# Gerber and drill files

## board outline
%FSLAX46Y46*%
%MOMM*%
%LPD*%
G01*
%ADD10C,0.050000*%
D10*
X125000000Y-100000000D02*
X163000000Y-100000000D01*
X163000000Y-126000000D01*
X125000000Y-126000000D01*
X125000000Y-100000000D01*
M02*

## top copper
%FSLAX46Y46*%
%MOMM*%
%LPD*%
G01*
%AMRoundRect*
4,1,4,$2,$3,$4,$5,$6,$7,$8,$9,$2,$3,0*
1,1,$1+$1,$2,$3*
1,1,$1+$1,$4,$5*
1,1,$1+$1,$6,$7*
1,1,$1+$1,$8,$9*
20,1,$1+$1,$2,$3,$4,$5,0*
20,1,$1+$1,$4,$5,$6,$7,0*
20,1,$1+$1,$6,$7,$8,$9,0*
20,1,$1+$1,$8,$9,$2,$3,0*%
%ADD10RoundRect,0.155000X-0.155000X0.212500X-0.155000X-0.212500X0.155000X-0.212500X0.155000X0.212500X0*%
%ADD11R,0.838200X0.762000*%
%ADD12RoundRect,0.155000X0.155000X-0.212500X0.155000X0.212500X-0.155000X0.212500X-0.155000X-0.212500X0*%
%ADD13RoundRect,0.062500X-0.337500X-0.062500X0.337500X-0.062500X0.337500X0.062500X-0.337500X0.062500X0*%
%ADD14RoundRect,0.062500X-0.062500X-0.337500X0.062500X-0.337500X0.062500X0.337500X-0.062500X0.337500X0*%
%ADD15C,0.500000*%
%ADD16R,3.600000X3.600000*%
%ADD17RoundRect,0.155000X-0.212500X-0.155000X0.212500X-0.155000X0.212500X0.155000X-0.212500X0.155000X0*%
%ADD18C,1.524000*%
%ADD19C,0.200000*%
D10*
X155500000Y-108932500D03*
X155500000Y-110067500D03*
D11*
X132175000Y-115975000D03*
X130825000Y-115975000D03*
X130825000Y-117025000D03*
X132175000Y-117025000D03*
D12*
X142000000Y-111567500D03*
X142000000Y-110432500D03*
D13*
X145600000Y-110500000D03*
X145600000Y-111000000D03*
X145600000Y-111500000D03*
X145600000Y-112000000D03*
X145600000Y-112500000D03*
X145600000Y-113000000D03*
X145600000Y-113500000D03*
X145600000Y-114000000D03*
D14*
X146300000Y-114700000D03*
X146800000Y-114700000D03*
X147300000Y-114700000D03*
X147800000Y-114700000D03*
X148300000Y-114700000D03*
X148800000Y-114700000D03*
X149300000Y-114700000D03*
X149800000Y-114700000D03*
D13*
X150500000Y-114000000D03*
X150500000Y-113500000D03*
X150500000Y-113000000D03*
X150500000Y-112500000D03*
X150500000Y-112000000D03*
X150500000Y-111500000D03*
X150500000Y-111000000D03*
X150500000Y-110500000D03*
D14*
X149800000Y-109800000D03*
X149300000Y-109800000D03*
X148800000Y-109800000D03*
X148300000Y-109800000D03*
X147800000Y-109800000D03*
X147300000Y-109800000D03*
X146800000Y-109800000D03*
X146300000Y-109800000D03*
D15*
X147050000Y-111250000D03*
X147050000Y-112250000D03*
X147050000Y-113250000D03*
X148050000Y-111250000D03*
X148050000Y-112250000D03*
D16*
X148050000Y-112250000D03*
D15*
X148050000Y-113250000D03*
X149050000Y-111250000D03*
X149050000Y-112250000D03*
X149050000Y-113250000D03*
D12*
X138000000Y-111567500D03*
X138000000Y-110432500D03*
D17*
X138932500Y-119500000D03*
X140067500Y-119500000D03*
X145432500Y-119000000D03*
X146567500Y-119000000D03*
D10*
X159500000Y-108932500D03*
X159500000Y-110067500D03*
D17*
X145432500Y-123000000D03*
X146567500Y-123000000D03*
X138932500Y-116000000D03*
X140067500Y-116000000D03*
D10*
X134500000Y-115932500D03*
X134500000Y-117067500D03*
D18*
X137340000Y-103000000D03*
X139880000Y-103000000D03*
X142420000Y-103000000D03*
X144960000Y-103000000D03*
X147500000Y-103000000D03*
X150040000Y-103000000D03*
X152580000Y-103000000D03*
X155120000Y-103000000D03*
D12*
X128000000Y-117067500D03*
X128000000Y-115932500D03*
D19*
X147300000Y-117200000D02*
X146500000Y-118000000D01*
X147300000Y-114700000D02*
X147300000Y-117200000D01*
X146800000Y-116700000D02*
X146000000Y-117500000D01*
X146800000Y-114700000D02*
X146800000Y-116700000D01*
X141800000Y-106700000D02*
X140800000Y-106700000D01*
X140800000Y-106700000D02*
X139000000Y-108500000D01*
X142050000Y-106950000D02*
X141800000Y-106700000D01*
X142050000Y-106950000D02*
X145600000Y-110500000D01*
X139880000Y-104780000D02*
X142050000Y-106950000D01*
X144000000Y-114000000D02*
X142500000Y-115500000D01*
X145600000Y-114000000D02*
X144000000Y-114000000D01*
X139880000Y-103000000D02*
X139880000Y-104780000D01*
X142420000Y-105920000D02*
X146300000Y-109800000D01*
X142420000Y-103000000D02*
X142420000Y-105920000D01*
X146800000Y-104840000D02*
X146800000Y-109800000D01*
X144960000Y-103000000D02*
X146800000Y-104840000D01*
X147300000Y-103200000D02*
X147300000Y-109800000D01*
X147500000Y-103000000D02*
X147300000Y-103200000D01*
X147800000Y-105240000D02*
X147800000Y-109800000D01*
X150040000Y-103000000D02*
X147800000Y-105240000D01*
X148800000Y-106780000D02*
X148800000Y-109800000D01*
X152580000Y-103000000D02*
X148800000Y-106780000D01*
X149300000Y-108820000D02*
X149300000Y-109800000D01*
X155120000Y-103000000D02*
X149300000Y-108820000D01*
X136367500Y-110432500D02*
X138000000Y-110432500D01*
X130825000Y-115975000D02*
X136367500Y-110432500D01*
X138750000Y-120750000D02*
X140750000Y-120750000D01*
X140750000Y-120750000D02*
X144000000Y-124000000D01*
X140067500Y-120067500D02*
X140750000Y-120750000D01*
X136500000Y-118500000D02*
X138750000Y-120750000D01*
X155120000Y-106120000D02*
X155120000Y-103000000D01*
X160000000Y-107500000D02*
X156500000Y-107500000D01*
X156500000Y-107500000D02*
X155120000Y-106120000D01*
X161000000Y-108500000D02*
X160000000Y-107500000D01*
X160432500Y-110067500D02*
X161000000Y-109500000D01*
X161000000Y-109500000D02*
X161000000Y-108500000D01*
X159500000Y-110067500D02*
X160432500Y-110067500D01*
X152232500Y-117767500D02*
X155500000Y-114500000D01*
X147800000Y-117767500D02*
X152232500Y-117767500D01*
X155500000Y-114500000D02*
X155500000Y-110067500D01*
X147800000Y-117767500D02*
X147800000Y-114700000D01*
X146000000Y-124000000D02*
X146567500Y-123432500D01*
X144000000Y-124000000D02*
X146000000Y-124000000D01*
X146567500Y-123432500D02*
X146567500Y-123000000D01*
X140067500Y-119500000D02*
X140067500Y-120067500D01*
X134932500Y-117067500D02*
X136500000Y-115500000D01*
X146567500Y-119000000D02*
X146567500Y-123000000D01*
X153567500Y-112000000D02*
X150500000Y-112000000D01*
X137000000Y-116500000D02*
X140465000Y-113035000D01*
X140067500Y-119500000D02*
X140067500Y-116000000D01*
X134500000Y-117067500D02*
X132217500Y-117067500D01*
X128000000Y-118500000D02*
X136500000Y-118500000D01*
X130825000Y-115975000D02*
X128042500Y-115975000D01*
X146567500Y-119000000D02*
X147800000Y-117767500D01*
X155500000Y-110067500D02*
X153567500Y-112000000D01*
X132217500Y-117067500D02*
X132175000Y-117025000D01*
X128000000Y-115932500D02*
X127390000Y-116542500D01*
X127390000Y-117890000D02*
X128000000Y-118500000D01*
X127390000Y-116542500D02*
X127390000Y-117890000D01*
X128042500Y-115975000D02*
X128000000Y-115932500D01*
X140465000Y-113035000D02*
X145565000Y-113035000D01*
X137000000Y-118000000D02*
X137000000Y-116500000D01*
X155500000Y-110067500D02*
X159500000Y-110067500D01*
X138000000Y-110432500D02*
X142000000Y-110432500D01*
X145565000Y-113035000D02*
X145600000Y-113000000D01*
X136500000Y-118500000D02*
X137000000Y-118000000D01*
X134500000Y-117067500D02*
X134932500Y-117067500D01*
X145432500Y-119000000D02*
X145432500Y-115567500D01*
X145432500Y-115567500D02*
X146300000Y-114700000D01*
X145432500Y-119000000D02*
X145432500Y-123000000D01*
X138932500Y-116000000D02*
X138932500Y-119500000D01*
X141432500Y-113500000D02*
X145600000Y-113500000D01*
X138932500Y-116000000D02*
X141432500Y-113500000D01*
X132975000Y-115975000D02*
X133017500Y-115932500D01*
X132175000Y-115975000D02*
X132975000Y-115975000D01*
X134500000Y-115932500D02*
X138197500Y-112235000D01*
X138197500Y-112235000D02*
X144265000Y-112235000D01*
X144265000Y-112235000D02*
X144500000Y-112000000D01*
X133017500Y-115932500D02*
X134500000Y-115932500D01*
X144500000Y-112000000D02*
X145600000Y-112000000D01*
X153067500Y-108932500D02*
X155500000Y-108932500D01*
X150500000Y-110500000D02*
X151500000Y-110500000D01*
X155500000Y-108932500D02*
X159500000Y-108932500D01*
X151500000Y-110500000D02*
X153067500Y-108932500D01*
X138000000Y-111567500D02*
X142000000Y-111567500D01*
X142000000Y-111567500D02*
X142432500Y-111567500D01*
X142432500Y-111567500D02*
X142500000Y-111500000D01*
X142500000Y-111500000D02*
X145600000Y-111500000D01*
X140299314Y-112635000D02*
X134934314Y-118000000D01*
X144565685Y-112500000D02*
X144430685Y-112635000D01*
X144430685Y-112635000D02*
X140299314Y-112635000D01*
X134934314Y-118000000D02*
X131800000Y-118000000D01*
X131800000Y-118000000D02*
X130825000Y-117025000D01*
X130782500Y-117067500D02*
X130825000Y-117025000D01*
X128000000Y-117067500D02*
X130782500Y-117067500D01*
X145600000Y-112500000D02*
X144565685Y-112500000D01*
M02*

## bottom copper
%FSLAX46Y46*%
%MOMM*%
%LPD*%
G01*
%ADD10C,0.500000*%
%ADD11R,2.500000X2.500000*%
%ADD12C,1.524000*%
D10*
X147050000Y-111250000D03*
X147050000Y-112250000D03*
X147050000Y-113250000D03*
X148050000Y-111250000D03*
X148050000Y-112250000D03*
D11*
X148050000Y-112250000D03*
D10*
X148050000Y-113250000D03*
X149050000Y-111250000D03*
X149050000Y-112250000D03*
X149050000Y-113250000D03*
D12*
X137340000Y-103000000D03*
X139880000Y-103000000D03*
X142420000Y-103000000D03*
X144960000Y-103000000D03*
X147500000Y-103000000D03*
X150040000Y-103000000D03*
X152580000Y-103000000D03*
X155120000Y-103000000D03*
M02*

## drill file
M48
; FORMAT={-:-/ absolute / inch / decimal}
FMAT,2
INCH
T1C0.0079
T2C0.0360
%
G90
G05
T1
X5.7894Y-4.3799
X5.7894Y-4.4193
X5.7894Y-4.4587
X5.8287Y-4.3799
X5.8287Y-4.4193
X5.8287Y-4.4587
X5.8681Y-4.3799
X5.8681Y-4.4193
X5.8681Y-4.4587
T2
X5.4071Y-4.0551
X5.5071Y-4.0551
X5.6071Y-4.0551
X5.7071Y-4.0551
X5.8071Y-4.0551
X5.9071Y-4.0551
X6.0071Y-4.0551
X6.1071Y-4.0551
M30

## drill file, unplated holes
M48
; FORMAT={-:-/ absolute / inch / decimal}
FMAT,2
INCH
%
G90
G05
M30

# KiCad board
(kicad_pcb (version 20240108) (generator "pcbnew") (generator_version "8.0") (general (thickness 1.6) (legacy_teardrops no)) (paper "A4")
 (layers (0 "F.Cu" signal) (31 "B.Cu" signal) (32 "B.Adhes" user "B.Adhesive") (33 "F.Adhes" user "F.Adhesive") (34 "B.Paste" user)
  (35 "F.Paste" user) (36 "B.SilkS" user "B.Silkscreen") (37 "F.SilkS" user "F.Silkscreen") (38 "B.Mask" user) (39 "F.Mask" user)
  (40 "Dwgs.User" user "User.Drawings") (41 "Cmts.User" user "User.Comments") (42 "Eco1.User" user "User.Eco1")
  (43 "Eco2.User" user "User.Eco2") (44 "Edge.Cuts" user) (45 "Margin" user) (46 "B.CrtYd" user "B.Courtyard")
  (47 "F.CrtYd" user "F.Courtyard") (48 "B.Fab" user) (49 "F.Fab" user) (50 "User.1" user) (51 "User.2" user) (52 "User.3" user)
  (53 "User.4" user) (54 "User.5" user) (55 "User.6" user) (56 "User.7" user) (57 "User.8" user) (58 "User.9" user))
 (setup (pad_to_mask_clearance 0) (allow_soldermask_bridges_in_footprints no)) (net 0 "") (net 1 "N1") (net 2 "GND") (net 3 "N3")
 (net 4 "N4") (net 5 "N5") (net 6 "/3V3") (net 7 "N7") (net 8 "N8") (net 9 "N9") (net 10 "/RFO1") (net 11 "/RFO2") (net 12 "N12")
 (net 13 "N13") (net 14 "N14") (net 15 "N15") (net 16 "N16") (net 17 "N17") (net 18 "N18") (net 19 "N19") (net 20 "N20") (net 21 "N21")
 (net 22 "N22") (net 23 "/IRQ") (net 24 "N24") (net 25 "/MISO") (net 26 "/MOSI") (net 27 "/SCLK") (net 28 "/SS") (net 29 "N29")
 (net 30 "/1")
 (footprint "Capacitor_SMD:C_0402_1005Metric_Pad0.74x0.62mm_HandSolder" (layer "F.Cu") (at 155.5 109.5 -90)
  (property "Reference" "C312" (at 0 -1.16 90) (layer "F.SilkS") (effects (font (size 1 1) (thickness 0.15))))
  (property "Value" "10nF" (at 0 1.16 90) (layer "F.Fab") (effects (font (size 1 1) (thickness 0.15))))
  (pad "1" smd roundrect (at -0.5675 0 270) (size 0.735 0.62) (layers "F.Cu" "F.Paste" "F.Mask") (roundrect_rratio 0.25) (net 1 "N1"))
  (pad "2" smd roundrect (at 0.5675 0 270) (size 0.735 0.62) (layers "F.Cu" "F.Paste" "F.Mask") (roundrect_rratio 0.25) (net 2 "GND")))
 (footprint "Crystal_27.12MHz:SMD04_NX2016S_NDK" (layer "F.Cu") (at 131.5 116.5 -90)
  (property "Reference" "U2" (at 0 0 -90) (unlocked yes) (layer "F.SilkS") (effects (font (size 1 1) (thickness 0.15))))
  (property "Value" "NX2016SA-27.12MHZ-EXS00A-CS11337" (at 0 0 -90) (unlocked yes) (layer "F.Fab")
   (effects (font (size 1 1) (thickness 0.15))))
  (pad "1" smd rect (at -0.525 -0.675 270) (size 0.762 0.8382) (layers "F.Cu" "F.Paste" "F.Mask") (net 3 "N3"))
  (pad "2" smd rect (at -0.525 0.675 270) (size 0.762 0.8382) (layers "F.Cu" "F.Paste" "F.Mask") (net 2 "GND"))
  (pad "3" smd rect (at 0.525 0.675 270) (size 0.762 0.8382) (layers "F.Cu" "F.Paste" "F.Mask") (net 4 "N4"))
  (pad "4" smd rect (at 0.525 -0.675 270) (size 0.762 0.8382) (layers "F.Cu" "F.Paste" "F.Mask") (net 2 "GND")))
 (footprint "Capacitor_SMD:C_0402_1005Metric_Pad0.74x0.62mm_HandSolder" (layer "F.Cu") (at 142 111 90)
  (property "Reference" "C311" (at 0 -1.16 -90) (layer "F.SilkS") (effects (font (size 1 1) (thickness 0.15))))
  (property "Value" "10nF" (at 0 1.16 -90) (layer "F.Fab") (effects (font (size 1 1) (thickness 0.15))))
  (pad "1" smd roundrect (at -0.5675 0 90) (size 0.735 0.62) (layers "F.Cu" "F.Paste" "F.Mask") (roundrect_rratio 0.25) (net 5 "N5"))
  (pad "2" smd roundrect (at 0.5675 0 90) (size 0.735 0.62) (layers "F.Cu" "F.Paste" "F.Mask") (roundrect_rratio 0.25) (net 2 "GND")))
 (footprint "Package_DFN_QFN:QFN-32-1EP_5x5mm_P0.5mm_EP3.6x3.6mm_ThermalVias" (layer "F.Cu") (at 148.05 112.25)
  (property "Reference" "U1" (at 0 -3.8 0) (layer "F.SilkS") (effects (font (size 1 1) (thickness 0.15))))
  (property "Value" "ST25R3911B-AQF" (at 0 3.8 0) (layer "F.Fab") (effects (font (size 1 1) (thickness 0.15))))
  (pad "" smd custom (at -1.4 -1.4) (size 0.554596 0.554596) (layers "F.Paste") (options (clearance outline) (anchor circle)) (primitives))
  (pad "" smd custom (at -1.4 -0.5) (size 0.568298 0.568298) (layers "F.Paste") (options (clearance outline) (anchor circle)) (primitives))
  (pad "" smd custom (at -1.4 0.5) (size 0.568298 0.568298) (layers "F.Paste") (options (clearance outline) (anchor circle)) (primitives))
  (pad "" smd custom (at -1.4 1.4) (size 0.554596 0.554596) (layers "F.Paste") (options (clearance outline) (anchor circle)) (primitives))
  (pad "" smd custom (at -0.5 -1.4) (size 0.568298 0.568298) (layers "F.Paste") (options (clearance outline) (anchor circle)) (primitives))
  (pad "" smd roundrect (at -0.5 -0.5) (size 0.806226 0.806226) (layers "F.Paste") (roundrect_rratio 0.25))
  (pad "" smd roundrect (at -0.5 0.5) (size 0.806226 0.806226) (layers "F.Paste") (roundrect_rratio 0.25))
  (pad "" smd custom (at -0.5 1.4) (size 0.568298 0.568298) (layers "F.Paste") (options (clearance outline) (anchor circle)) (primitives))
  (pad "" smd custom (at 0.5 -1.4) (size 0.568298 0.568298) (layers "F.Paste") (options (clearance outline) (anchor circle)) (primitives))
  (pad "" smd roundrect (at 0.5 -0.5) (size 0.806226 0.806226) (layers "F.Paste") (roundrect_rratio 0.25))
  (pad "" smd roundrect (at 0.5 0.5) (size 0.806226 0.806226) (layers "F.Paste") (roundrect_rratio 0.25))
  (pad "" smd custom (at 0.5 1.4) (size 0.568298 0.568298) (layers "F.Paste") (options (clearance outline) (anchor circle)) (primitives))
  (pad "" smd custom (at 1.4 -1.4) (size 0.554596 0.554596) (layers "F.Paste") (options (clearance outline) (anchor circle)) (primitives))
  (pad "" smd custom (at 1.4 -0.5) (size 0.568298 0.568298) (layers "F.Paste") (options (clearance outline) (anchor circle)) (primitives))
  (pad "" smd custom (at 1.4 0.5) (size 0.568298 0.568298) (layers "F.Paste") (options (clearance outline) (anchor circle)) (primitives))
  (pad "" smd custom (at 1.4 1.4) (size 0.554596 0.554596) (layers "F.Paste") (options (clearance outline) (anchor circle)) (primitives))
  (pad "1" smd roundrect (at -2.45 -1.75) (size 0.8 0.25) (layers "F.Cu" "F.Paste" "F.Mask") (roundrect_rratio 0.25) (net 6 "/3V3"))
  (pad "2" smd roundrect (at -2.45 -1.25) (size 0.8 0.25) (layers "F.Cu" "F.Paste" "F.Mask") (roundrect_rratio 0.25) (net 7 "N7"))
  (pad "3" smd roundrect (at -2.45 -0.75) (size 0.8 0.25) (layers "F.Cu" "F.Paste" "F.Mask") (roundrect_rratio 0.25) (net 5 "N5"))
  (pad "4" smd roundrect (at -2.45 -0.25) (size 0.8 0.25) (layers "F.Cu" "F.Paste" "F.Mask") (roundrect_rratio 0.25) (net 3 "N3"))
  (pad "5" smd roundrect (at -2.45 0.25) (size 0.8 0.25) (layers "F.Cu" "F.Paste" "F.Mask") (roundrect_rratio 0.25) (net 4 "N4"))
  (pad "6" smd roundrect (at -2.45 0.75) (size 0.8 0.25) (layers "F.Cu" "F.Paste" "F.Mask") (roundrect_rratio 0.25) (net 2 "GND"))
  (pad "7" smd roundrect (at -2.45 1.25) (size 0.8 0.25) (layers "F.Cu" "F.Paste" "F.Mask") (roundrect_rratio 0.25) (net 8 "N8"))
  (pad "8" smd roundrect (at -2.45 1.75) (size 0.8 0.25) (layers "F.Cu" "F.Paste" "F.Mask") (roundrect_rratio 0.25) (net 6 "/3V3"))
  (pad "9" smd roundrect (at -1.75 2.45) (size 0.25 0.8) (layers "F.Cu" "F.Paste" "F.Mask") (roundrect_rratio 0.25) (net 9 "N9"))
  (pad "10" smd roundrect (at -1.25 2.45) (size 0.25 0.8) (layers "F.Cu" "F.Paste" "F.Mask") (roundrect_rratio 0.25) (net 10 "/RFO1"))
  (pad "11" smd roundrect (at -0.75 2.45) (size 0.25 0.8) (layers "F.Cu" "F.Paste" "F.Mask") (roundrect_rratio 0.25) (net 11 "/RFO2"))
  (pad "12" smd roundrect (at -0.25 2.45) (size 0.25 0.8) (layers "F.Cu" "F.Paste" "F.Mask") (roundrect_rratio 0.25) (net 2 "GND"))
  (pad "13" smd roundrect (at 0.25 2.45) (size 0.25 0.8) (layers "F.Cu" "F.Paste" "F.Mask") (roundrect_rratio 0.25) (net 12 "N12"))
  (pad "14" smd roundrect (at 0.75 2.45) (size 0.25 0.8) (layers "F.Cu" "F.Paste" "F.Mask") (roundrect_rratio 0.25) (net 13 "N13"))
  (pad "15" smd roundrect (at 1.25 2.45) (size 0.25 0.8) (layers "F.Cu" "F.Paste" "F.Mask") (roundrect_rratio 0.25) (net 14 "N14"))
  (pad "16" smd roundrect (at 1.75 2.45) (size 0.25 0.8) (layers "F.Cu" "F.Paste" "F.Mask") (roundrect_rratio 0.25) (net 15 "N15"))
  (pad "17" smd roundrect (at 2.45 1.75) (size 0.8 0.25) (layers "F.Cu" "F.Paste" "F.Mask") (roundrect_rratio 0.25) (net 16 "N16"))
  (pad "18" smd roundrect (at 2.45 1.25) (size 0.8 0.25) (layers "F.Cu" "F.Paste" "F.Mask") (roundrect_rratio 0.25) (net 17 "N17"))
  (pad "19" smd roundrect (at 2.45 0.75) (size 0.8 0.25) (layers "F.Cu" "F.Paste" "F.Mask") (roundrect_rratio 0.25) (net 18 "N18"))
  (pad "20" smd roundrect (at 2.45 0.25) (size 0.8 0.25) (layers "F.Cu" "F.Paste" "F.Mask") (roundrect_rratio 0.25) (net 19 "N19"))
  (pad "21" smd roundrect (at 2.45 -0.25) (size 0.8 0.25) (layers "F.Cu" "F.Paste" "F.Mask") (roundrect_rratio 0.25) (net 2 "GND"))
  (pad "22" smd roundrect (at 2.45 -0.75) (size 0.8 0.25) (layers "F.Cu" "F.Paste" "F.Mask") (roundrect_rratio 0.25) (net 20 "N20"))
  (pad "23" smd roundrect (at 2.45 -1.25) (size 0.8 0.25) (layers "F.Cu" "F.Paste" "F.Mask") (roundrect_rratio 0.25) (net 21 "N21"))
  (pad "24" smd roundrect (at 2.45 -1.75) (size 0.8 0.25) (layers "F.Cu" "F.Paste" "F.Mask") (roundrect_rratio 0.25) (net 1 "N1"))
  (pad "25" smd roundrect (at 1.75 -2.45) (size 0.25 0.8) (layers "F.Cu" "F.Paste" "F.Mask") (roundrect_rratio 0.25) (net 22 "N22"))
  (pad "26" smd roundrect (at 1.25 -2.45) (size 0.25 0.8) (layers "F.Cu" "F.Paste" "F.Mask") (roundrect_rratio 0.25) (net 2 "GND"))
  (pad "27" smd roundrect (at 0.75 -2.45) (size 0.25 0.8) (layers "F.Cu" "F.Paste" "F.Mask") (roundrect_rratio 0.25) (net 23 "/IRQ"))
  (pad "28" smd roundrect (at 0.25 -2.45) (size 0.25 0.8) (layers "F.Cu" "F.Paste" "F.Mask") (roundrect_rratio 0.25) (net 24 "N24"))
  (pad "29" smd roundrect (at -0.25 -2.45) (size 0.25 0.8) (layers "F.Cu" "F.Paste" "F.Mask") (roundrect_rratio 0.25) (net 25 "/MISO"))
  (pad "30" smd roundrect (at -0.75 -2.45) (size 0.25 0.8) (layers "F.Cu" "F.Paste" "F.Mask") (roundrect_rratio 0.25) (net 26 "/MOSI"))
  (pad "31" smd roundrect (at -1.25 -2.45) (size 0.25 0.8) (layers "F.Cu" "F.Paste" "F.Mask") (roundrect_rratio 0.25) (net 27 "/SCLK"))
  (pad "32" smd roundrect (at -1.75 -2.45) (size 0.25 0.8) (layers "F.Cu" "F.Paste" "F.Mask") (roundrect_rratio 0.25) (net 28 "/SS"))
  (pad "33" thru_hole circle (at -1 -1) (size 0.5 0.5) (drill 0.2) (layers "*.Cu") (remove_unused_layers no) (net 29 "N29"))
  (pad "33" thru_hole circle (at -1 0) (size 0.5 0.5) (drill 0.2) (layers "*.Cu") (remove_unused_layers no) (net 29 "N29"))
  (pad "33" thru_hole circle (at -1 1) (size 0.5 0.5) (drill 0.2) (layers "*.Cu") (remove_unused_layers no) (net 29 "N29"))
  (pad "33" thru_hole circle (at 0 -1) (size 0.5 0.5) (drill 0.2) (layers "*.Cu") (remove_unused_layers no) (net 29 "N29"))
  (pad "33" thru_hole circle (at 0 0) (size 0.5 0.5) (drill 0.2) (layers "*.Cu") (remove_unused_layers no) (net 29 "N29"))
  (pad "33" smd rect (at 0 0) (size 2.5 2.5) (layers "B.Cu") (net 29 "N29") (zone_connect 2))
  (pad "33" smd rect (at 0 0) (size 3.6 3.6) (layers "F.Cu" "F.Mask") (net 29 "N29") (zone_connect 2))
  (pad "33" thru_hole circle (at 0 1) (size 0.5 0.5) (drill 0.2) (layers "*.Cu") (remove_unused_layers no) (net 29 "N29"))
  (pad "33" thru_hole circle (at 1 -1) (size 0.5 0.5) (drill 0.2) (layers "*.Cu") (remove_unused_layers no) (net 29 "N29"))
  (pad "33" thru_hole circle (at 1 0) (size 0.5 0.5) (drill 0.2) (layers "*.Cu") (remove_unused_layers no) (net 29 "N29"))
  (pad "33" thru_hole circle (at 1 1) (size 0.5 0.5) (drill 0.2) (layers "*.Cu") (remove_unused_layers no) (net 29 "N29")))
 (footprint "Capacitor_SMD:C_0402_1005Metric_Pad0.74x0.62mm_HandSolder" (layer "F.Cu") (at 138 111 90)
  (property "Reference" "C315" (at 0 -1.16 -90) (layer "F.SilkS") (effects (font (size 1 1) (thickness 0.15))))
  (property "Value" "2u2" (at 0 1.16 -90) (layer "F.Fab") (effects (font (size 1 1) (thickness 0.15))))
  (pad "1" smd roundrect (at -0.5675 0 90) (size 0.735 0.62) (layers "F.Cu" "F.Paste" "F.Mask") (roundrect_rratio 0.25) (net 5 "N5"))
  (pad "2" smd roundrect (at 0.5675 0 90) (size 0.735 0.62) (layers "F.Cu" "F.Paste" "F.Mask") (roundrect_rratio 0.25) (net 2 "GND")))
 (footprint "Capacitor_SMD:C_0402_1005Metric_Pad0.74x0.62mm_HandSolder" (layer "F.Cu") (at 139.5 119.5)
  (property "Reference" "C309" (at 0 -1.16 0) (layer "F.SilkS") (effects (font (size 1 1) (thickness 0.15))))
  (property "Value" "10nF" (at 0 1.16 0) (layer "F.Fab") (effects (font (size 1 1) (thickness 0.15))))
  (pad "1" smd roundrect (at -0.5675 0) (size 0.735 0.62) (layers "F.Cu" "F.Paste" "F.Mask") (roundrect_rratio 0.25) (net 8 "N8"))
  (pad "2" smd roundrect (at 0.5675 0) (size 0.735 0.62) (layers "F.Cu" "F.Paste" "F.Mask") (roundrect_rratio 0.25) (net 2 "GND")))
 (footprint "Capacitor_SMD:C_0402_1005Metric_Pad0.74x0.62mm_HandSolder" (layer "F.Cu") (at 146 119)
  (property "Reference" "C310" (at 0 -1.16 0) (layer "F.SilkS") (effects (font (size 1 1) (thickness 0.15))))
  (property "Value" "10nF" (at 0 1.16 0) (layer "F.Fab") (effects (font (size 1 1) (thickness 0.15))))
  (pad "1" smd roundrect (at -0.5675 0) (size 0.735 0.62) (layers "F.Cu" "F.Paste" "F.Mask") (roundrect_rratio 0.25) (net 9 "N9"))
  (pad "2" smd roundrect (at 0.5675 0) (size 0.735 0.62) (layers "F.Cu" "F.Paste" "F.Mask") (roundrect_rratio 0.25) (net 2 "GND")))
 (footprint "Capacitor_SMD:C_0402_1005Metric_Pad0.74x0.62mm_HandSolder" (layer "F.Cu") (at 159.5 109.5 -90)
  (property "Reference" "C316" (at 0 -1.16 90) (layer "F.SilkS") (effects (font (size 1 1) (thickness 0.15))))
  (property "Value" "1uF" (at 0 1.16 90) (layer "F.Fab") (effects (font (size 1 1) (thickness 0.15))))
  (pad "1" smd roundrect (at -0.5675 0 270) (size 0.735 0.62) (layers "F.Cu" "F.Paste" "F.Mask") (roundrect_rratio 0.25) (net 1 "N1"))
  (pad "2" smd roundrect (at 0.5675 0 270) (size 0.735 0.62) (layers "F.Cu" "F.Paste" "F.Mask") (roundrect_rratio 0.25) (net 2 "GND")))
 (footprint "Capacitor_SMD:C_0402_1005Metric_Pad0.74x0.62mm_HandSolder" (layer "F.Cu") (at 146 123)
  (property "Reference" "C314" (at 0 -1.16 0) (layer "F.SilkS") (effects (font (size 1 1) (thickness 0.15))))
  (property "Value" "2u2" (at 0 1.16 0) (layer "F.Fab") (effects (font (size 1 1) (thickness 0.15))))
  (pad "1" smd roundrect (at -0.5675 0) (size 0.735 0.62) (layers "F.Cu" "F.Paste" "F.Mask") (roundrect_rratio 0.25) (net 9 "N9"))
  (pad "2" smd roundrect (at 0.5675 0) (size 0.735 0.62) (layers "F.Cu" "F.Paste" "F.Mask") (roundrect_rratio 0.25) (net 2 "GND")))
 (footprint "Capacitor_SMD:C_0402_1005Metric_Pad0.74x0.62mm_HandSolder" (layer "F.Cu") (at 139.5 116)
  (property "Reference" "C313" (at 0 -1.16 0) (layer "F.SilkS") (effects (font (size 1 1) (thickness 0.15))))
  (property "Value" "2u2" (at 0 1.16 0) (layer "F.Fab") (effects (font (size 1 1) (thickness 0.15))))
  (pad "1" smd roundrect (at -0.5675 0) (size 0.735 0.62) (layers "F.Cu" "F.Paste" "F.Mask") (roundrect_rratio 0.25) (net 8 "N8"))
  (pad "2" smd roundrect (at 0.5675 0) (size 0.735 0.62) (layers "F.Cu" "F.Paste" "F.Mask") (roundrect_rratio 0.25) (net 2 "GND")))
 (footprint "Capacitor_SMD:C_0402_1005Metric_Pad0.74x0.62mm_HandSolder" (layer "F.Cu") (at 134.5 116.5 -90)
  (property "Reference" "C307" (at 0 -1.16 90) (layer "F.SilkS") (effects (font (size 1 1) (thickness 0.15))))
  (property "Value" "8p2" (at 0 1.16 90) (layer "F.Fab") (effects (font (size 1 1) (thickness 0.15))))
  (pad "1" smd roundrect (at -0.5675 0 270) (size 0.735 0.62) (layers "F.Cu" "F.Paste" "F.Mask") (roundrect_rratio 0.25) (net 3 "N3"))
  (pad "2" smd roundrect (at 0.5675 0 270) (size 0.735 0.62) (layers "F.Cu" "F.Paste" "F.Mask") (roundrect_rratio 0.25) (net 2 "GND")))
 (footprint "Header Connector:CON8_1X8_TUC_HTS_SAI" (layer "F.Cu") (at 146.23 103)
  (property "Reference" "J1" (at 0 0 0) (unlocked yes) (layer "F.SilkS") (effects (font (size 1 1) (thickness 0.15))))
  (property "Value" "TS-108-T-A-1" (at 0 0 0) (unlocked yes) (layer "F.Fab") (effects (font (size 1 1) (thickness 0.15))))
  (pad "1" thru_hole circle (at -8.89 0 90) (size 1.524 1.524) (drill 0.9144) (layers "*.Cu" "*.Mask") (remove_unused_layers no)
   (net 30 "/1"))
  (pad "2" thru_hole circle (at -6.35 0 90) (size 1.524 1.524) (drill 0.9144) (layers "*.Cu" "*.Mask") (remove_unused_layers no)
   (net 6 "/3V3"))
  (pad "3" thru_hole circle (at -3.81 0 90) (size 1.524 1.524) (drill 0.9144) (layers "*.Cu" "*.Mask") (remove_unused_layers no)
   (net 28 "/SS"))
  (pad "4" thru_hole circle (at -1.27 0 90) (size 1.524 1.524) (drill 0.9144) (layers "*.Cu" "*.Mask") (remove_unused_layers no)
   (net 27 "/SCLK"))
  (pad "5" thru_hole circle (at 1.27 0 90) (size 1.524 1.524) (drill 0.9144) (layers "*.Cu" "*.Mask") (remove_unused_layers no)
   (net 26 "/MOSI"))
  (pad "6" thru_hole circle (at 3.81 0 90) (size 1.524 1.524) (drill 0.9144) (layers "*.Cu" "*.Mask") (remove_unused_layers no)
   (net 25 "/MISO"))
  (pad "7" thru_hole circle (at 6.35 0 90) (size 1.524 1.524) (drill 0.9144) (layers "*.Cu" "*.Mask") (remove_unused_layers no)
   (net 23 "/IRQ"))
  (pad "8" thru_hole circle (at 8.89 0 90) (size 1.524 1.524) (drill 0.9144) (layers "*.Cu" "*.Mask") (remove_unused_layers no)
   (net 2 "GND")))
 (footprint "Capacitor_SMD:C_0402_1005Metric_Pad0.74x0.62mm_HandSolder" (layer "F.Cu") (at 128 116.5 90)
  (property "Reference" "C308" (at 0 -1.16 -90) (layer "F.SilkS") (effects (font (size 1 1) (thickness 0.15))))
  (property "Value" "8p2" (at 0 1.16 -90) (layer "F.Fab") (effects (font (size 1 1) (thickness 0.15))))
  (pad "1" smd roundrect (at -0.5675 0 90) (size 0.735 0.62) (layers "F.Cu" "F.Paste" "F.Mask") (roundrect_rratio 0.25) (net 4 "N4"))
  (pad "2" smd roundrect (at 0.5675 0 90) (size 0.735 0.62) (layers "F.Cu" "F.Paste" "F.Mask") (roundrect_rratio 0.25) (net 2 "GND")))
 (gr_rect (start 125 100) (end 163 126) (stroke (width 0.05) (type default)) (fill none) (layer "Edge.Cuts"))
 (segment (start 147.5 103) (end 147.3 103.2) (width 0.2) (layer "F.Cu") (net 26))
 (segment (start 147.3 103.2) (end 147.3 109.8) (width 0.2) (layer "F.Cu") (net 26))
 (segment (start 144 114) (end 142.5 115.5) (width 0.2) (layer "F.Cu") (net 6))
 (segment (start 139.88 103) (end 139.88 104.78) (width 0.2) (layer "F.Cu") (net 6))
 (segment (start 140.8 106.7) (end 139 108.5) (width 0.2) (layer "F.Cu") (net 6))
 (segment (start 139.88 104.78) (end 142.05 106.95) (width 0.2) (layer "F.Cu") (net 6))
 (segment (start 141.8 106.7) (end 140.8 106.7) (width 0.2) (layer "F.Cu") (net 6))
 (segment (start 142.05 106.95) (end 141.8 106.7) (width 0.2) (layer "F.Cu") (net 6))
 (segment (start 145.6 114) (end 144 114) (width 0.2) (layer "F.Cu") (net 6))
 (segment (start 142.05 106.95) (end 145.6 110.5) (width 0.2) (layer "F.Cu") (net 6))
 (segment (start 152.58 103) (end 148.8 106.78) (width 0.2) (layer "F.Cu") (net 23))
 (segment (start 148.8 106.78) (end 148.8 109.8) (width 0.2) (layer "F.Cu") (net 23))
 (segment (start 136.5 118.5) (end 138.75 120.75) (width 0.2) (layer "F.Cu") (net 2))
 (segment (start 134.9325 117.0675) (end 136.5 115.5) (width 0.2) (layer "F.Cu") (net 2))
 (segment (start 146.5675 119) (end 146.5675 123) (width 0.2) (layer "F.Cu") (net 2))
 (segment (start 155.12 106.12) (end 155.12 103) (width 0.2) (layer "F.Cu") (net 2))
 (segment (start 153.5675 112) (end 150.5 112) (width 0.2) (layer "F.Cu") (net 2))
 (segment (start 160.4325 110.0675) (end 161 109.5) (width 0.2) (layer "F.Cu") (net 2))
 (segment (start 137 116.5) (end 140.465 113.035) (width 0.2) (layer "F.Cu") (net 2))
 (segment (start 146 124) (end 146.5675 123.4325) (width 0.2) (layer "F.Cu") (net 2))
 (segment (start 147.8 117.7675) (end 152.2325 117.7675) (width 0.2) (layer "F.Cu") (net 2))
 (segment (start 140.0675 119.5) (end 140.0675 116) (width 0.2) (layer "F.Cu") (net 2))
 (segment (start 140.0675 120.0675) (end 140.75 120.75) (width 0.2) (layer "F.Cu") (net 2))
 (segment (start 134.5 117.0675) (end 132.2175 117.0675) (width 0.2) (layer "F.Cu") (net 2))
 (segment (start 140.75 120.75) (end 144 124) (width 0.2) (layer "F.Cu") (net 2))
 (segment (start 160 107.5) (end 156.5 107.5) (width 0.2) (layer "F.Cu") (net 2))
 (segment (start 128 118.5) (end 136.5 118.5) (width 0.2) (layer "F.Cu") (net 2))
 (segment (start 130.825 115.975) (end 128.0425 115.975) (width 0.2) (layer "F.Cu") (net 2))
 (segment (start 146.5675 119) (end 147.8 117.7675) (width 0.2) (layer "F.Cu") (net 2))
 (segment (start 155.5 110.0675) (end 153.5675 112) (width 0.2) (layer "F.Cu") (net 2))
 (segment (start 140.0675 119.5) (end 140.0675 120.0675) (width 0.2) (layer "F.Cu") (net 2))
 (segment (start 155.12 103) (end 149.3 108.82) (width 0.2) (layer "F.Cu") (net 2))
 (segment (start 132.2175 117.0675) (end 132.175 117.025) (width 0.2) (layer "F.Cu") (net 2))
 (segment (start 149.3 108.82) (end 149.3 109.8) (width 0.2) (layer "F.Cu") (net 2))
 (segment (start 128 115.9325) (end 127.39 116.5425) (width 0.2) (layer "F.Cu") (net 2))
 (segment (start 159.5 110.0675) (end 160.4325 110.0675) (width 0.2) (layer "F.Cu") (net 2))
 (segment (start 138.75 120.75) (end 140.75 120.75) (width 0.2) (layer "F.Cu") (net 2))
 (segment (start 127.39 117.89) (end 128 118.5) (width 0.2) (layer "F.Cu") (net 2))
 (segment (start 127.39 116.5425) (end 127.39 117.89) (width 0.2) (layer "F.Cu") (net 2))
 (segment (start 161 109.5) (end 161 108.5) (width 0.2) (layer "F.Cu") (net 2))
 (segment (start 161 108.5) (end 160 107.5) (width 0.2) (layer "F.Cu") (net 2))
 (segment (start 144 124) (end 146 124) (width 0.2) (layer "F.Cu") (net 2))
 (segment (start 128.0425 115.975) (end 128 115.9325) (width 0.2) (layer "F.Cu") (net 2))
 (segment (start 140.465 113.035) (end 145.565 113.035) (width 0.2) (layer "F.Cu") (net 2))
 (segment (start 147.8 117.7675) (end 147.8 114.7) (width 0.2) (layer "F.Cu") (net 2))
 (segment (start 130.825 115.975) (end 136.3675 110.4325) (width 0.2) (layer "F.Cu") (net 2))
 (segment (start 137 118) (end 137 116.5) (width 0.2) (layer "F.Cu") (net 2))
 (segment (start 146.5675 123.4325) (end 146.5675 123) (width 0.2) (layer "F.Cu") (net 2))
 (segment (start 155.5 110.0675) (end 159.5 110.0675) (width 0.2) (layer "F.Cu") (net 2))
 (segment (start 138 110.4325) (end 142 110.4325) (width 0.2) (layer "F.Cu") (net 2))
 (segment (start 152.2325 117.7675) (end 155.5 114.5) (width 0.2) (layer "F.Cu") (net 2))
 (segment (start 145.565 113.035) (end 145.6 113) (width 0.2) (layer "F.Cu") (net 2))
 (segment (start 136.5 118.5) (end 137 118) (width 0.2) (layer "F.Cu") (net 2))
 (segment (start 156.5 107.5) (end 155.12 106.12) (width 0.2) (layer "F.Cu") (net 2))
 (segment (start 136.3675 110.4325) (end 138 110.4325) (width 0.2) (layer "F.Cu") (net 2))
 (segment (start 134.5 117.0675) (end 134.9325 117.0675) (width 0.2) (layer "F.Cu") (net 2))
 (segment (start 155.5 114.5) (end 155.5 110.0675) (width 0.2) (layer "F.Cu") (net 2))
 (segment (start 147.8 105.24) (end 147.8 109.8) (width 0.2) (layer "F.Cu") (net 25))
 (segment (start 150.04 103) (end 147.8 105.24) (width 0.2) (layer "F.Cu") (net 25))
 (segment (start 142.42 103) (end 142.42 105.92) (width 0.2) (layer "F.Cu") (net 28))
 (segment (start 142.42 105.92) (end 146.3 109.8) (width 0.2) (layer "F.Cu") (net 28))
 (segment (start 144.96 103) (end 146.8 104.84) (width 0.2) (layer "F.Cu") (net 27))
 (segment (start 146.8 104.84) (end 146.8 109.8) (width 0.2) (layer "F.Cu") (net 27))
 (segment (start 145.4325 119) (end 145.4325 115.5675) (width 0.2) (layer "F.Cu") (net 9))
 (segment (start 145.4325 115.5675) (end 146.3 114.7) (width 0.2) (layer "F.Cu") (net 9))
 (segment (start 145.4325 119) (end 145.4325 123) (width 0.2) (layer "F.Cu") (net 9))
 (segment (start 138.9325 116) (end 138.9325 119.5) (width 0.2) (layer "F.Cu") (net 8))
 (segment (start 141.4325 113.5) (end 145.6 113.5) (width 0.2) (layer "F.Cu") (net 8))
 (segment (start 138.9325 116) (end 141.4325 113.5) (width 0.2) (layer "F.Cu") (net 8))
 (segment (start 132.975 115.975) (end 133.0175 115.9325) (width 0.2) (layer "F.Cu") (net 3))
 (segment (start 132.175 115.975) (end 132.975 115.975) (width 0.2) (layer "F.Cu") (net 3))
 (segment (start 134.5 115.9325) (end 138.1975 112.235) (width 0.2) (layer "F.Cu") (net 3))
 (segment (start 138.1975 112.235) (end 144.265 112.235) (width 0.2) (layer "F.Cu") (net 3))
 (segment (start 144.265 112.235) (end 144.5 112) (width 0.2) (layer "F.Cu") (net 3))
 (segment (start 133.0175 115.9325) (end 134.5 115.9325) (width 0.2) (layer "F.Cu") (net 3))
 (segment (start 144.5 112) (end 145.6 112) (width 0.2) (layer "F.Cu") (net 3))
 (segment (start 153.0675 108.9325) (end 155.5 108.9325) (width 0.2) (layer "F.Cu") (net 1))
 (segment (start 150.5 110.5) (end 151.5 110.5) (width 0.2) (layer "F.Cu") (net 1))
 (segment (start 155.5 108.9325) (end 159.5 108.9325) (width 0.2) (layer "F.Cu") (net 1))
 (segment (start 151.5 110.5) (end 153.0675 108.9325) (width 0.2) (layer "F.Cu") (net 1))
 (segment (start 138 111.5675) (end 142 111.5675) (width 0.2) (layer "F.Cu") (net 5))
 (segment (start 142 111.5675) (end 142.4325 111.5675) (width 0.2) (layer "F.Cu") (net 5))
 (segment (start 142.4325 111.5675) (end 142.5 111.5) (width 0.2) (layer "F.Cu") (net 5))
 (segment (start 142.5 111.5) (end 145.6 111.5) (width 0.2) (layer "F.Cu") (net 5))
 (segment (start 147.3 117.2) (end 146.5 118) (width 0.2) (layer "F.Cu") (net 11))
 (segment (start 147.3 114.7) (end 147.3 117.2) (width 0.2) (layer "F.Cu") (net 11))
 (segment (start 146.8 116.7) (end 146 117.5) (width 0.2) (layer "F.Cu") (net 10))
 (segment (start 146.8 114.7) (end 146.8 116.7) (width 0.2) (layer "F.Cu") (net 10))
 (segment (start 140.299314 112.635) (end 134.934314 118) (width 0.2) (layer "F.Cu") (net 4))
 (segment (start 144.565685 112.5) (end 144.430685 112.635) (width 0.2) (layer "F.Cu") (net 4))
 (segment (start 144.430685 112.635) (end 140.299314 112.635) (width 0.2) (layer "F.Cu") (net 4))
 (segment (start 134.934314 118) (end 131.8 118) (width 0.2) (layer "F.Cu") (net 4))
 (segment (start 131.8 118) (end 130.825 117.025) (width 0.2) (layer "F.Cu") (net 4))
 (segment (start 130.7825 117.0675) (end 130.825 117.025) (width 0.2) (layer "F.Cu") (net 4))
 (segment (start 128 117.0675) (end 130.7825 117.0675) (width 0.2) (layer "F.Cu") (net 4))
 (segment (start 145.6 112.5) (end 144.565685 112.5) (width 0.2) (layer "F.Cu") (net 4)))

